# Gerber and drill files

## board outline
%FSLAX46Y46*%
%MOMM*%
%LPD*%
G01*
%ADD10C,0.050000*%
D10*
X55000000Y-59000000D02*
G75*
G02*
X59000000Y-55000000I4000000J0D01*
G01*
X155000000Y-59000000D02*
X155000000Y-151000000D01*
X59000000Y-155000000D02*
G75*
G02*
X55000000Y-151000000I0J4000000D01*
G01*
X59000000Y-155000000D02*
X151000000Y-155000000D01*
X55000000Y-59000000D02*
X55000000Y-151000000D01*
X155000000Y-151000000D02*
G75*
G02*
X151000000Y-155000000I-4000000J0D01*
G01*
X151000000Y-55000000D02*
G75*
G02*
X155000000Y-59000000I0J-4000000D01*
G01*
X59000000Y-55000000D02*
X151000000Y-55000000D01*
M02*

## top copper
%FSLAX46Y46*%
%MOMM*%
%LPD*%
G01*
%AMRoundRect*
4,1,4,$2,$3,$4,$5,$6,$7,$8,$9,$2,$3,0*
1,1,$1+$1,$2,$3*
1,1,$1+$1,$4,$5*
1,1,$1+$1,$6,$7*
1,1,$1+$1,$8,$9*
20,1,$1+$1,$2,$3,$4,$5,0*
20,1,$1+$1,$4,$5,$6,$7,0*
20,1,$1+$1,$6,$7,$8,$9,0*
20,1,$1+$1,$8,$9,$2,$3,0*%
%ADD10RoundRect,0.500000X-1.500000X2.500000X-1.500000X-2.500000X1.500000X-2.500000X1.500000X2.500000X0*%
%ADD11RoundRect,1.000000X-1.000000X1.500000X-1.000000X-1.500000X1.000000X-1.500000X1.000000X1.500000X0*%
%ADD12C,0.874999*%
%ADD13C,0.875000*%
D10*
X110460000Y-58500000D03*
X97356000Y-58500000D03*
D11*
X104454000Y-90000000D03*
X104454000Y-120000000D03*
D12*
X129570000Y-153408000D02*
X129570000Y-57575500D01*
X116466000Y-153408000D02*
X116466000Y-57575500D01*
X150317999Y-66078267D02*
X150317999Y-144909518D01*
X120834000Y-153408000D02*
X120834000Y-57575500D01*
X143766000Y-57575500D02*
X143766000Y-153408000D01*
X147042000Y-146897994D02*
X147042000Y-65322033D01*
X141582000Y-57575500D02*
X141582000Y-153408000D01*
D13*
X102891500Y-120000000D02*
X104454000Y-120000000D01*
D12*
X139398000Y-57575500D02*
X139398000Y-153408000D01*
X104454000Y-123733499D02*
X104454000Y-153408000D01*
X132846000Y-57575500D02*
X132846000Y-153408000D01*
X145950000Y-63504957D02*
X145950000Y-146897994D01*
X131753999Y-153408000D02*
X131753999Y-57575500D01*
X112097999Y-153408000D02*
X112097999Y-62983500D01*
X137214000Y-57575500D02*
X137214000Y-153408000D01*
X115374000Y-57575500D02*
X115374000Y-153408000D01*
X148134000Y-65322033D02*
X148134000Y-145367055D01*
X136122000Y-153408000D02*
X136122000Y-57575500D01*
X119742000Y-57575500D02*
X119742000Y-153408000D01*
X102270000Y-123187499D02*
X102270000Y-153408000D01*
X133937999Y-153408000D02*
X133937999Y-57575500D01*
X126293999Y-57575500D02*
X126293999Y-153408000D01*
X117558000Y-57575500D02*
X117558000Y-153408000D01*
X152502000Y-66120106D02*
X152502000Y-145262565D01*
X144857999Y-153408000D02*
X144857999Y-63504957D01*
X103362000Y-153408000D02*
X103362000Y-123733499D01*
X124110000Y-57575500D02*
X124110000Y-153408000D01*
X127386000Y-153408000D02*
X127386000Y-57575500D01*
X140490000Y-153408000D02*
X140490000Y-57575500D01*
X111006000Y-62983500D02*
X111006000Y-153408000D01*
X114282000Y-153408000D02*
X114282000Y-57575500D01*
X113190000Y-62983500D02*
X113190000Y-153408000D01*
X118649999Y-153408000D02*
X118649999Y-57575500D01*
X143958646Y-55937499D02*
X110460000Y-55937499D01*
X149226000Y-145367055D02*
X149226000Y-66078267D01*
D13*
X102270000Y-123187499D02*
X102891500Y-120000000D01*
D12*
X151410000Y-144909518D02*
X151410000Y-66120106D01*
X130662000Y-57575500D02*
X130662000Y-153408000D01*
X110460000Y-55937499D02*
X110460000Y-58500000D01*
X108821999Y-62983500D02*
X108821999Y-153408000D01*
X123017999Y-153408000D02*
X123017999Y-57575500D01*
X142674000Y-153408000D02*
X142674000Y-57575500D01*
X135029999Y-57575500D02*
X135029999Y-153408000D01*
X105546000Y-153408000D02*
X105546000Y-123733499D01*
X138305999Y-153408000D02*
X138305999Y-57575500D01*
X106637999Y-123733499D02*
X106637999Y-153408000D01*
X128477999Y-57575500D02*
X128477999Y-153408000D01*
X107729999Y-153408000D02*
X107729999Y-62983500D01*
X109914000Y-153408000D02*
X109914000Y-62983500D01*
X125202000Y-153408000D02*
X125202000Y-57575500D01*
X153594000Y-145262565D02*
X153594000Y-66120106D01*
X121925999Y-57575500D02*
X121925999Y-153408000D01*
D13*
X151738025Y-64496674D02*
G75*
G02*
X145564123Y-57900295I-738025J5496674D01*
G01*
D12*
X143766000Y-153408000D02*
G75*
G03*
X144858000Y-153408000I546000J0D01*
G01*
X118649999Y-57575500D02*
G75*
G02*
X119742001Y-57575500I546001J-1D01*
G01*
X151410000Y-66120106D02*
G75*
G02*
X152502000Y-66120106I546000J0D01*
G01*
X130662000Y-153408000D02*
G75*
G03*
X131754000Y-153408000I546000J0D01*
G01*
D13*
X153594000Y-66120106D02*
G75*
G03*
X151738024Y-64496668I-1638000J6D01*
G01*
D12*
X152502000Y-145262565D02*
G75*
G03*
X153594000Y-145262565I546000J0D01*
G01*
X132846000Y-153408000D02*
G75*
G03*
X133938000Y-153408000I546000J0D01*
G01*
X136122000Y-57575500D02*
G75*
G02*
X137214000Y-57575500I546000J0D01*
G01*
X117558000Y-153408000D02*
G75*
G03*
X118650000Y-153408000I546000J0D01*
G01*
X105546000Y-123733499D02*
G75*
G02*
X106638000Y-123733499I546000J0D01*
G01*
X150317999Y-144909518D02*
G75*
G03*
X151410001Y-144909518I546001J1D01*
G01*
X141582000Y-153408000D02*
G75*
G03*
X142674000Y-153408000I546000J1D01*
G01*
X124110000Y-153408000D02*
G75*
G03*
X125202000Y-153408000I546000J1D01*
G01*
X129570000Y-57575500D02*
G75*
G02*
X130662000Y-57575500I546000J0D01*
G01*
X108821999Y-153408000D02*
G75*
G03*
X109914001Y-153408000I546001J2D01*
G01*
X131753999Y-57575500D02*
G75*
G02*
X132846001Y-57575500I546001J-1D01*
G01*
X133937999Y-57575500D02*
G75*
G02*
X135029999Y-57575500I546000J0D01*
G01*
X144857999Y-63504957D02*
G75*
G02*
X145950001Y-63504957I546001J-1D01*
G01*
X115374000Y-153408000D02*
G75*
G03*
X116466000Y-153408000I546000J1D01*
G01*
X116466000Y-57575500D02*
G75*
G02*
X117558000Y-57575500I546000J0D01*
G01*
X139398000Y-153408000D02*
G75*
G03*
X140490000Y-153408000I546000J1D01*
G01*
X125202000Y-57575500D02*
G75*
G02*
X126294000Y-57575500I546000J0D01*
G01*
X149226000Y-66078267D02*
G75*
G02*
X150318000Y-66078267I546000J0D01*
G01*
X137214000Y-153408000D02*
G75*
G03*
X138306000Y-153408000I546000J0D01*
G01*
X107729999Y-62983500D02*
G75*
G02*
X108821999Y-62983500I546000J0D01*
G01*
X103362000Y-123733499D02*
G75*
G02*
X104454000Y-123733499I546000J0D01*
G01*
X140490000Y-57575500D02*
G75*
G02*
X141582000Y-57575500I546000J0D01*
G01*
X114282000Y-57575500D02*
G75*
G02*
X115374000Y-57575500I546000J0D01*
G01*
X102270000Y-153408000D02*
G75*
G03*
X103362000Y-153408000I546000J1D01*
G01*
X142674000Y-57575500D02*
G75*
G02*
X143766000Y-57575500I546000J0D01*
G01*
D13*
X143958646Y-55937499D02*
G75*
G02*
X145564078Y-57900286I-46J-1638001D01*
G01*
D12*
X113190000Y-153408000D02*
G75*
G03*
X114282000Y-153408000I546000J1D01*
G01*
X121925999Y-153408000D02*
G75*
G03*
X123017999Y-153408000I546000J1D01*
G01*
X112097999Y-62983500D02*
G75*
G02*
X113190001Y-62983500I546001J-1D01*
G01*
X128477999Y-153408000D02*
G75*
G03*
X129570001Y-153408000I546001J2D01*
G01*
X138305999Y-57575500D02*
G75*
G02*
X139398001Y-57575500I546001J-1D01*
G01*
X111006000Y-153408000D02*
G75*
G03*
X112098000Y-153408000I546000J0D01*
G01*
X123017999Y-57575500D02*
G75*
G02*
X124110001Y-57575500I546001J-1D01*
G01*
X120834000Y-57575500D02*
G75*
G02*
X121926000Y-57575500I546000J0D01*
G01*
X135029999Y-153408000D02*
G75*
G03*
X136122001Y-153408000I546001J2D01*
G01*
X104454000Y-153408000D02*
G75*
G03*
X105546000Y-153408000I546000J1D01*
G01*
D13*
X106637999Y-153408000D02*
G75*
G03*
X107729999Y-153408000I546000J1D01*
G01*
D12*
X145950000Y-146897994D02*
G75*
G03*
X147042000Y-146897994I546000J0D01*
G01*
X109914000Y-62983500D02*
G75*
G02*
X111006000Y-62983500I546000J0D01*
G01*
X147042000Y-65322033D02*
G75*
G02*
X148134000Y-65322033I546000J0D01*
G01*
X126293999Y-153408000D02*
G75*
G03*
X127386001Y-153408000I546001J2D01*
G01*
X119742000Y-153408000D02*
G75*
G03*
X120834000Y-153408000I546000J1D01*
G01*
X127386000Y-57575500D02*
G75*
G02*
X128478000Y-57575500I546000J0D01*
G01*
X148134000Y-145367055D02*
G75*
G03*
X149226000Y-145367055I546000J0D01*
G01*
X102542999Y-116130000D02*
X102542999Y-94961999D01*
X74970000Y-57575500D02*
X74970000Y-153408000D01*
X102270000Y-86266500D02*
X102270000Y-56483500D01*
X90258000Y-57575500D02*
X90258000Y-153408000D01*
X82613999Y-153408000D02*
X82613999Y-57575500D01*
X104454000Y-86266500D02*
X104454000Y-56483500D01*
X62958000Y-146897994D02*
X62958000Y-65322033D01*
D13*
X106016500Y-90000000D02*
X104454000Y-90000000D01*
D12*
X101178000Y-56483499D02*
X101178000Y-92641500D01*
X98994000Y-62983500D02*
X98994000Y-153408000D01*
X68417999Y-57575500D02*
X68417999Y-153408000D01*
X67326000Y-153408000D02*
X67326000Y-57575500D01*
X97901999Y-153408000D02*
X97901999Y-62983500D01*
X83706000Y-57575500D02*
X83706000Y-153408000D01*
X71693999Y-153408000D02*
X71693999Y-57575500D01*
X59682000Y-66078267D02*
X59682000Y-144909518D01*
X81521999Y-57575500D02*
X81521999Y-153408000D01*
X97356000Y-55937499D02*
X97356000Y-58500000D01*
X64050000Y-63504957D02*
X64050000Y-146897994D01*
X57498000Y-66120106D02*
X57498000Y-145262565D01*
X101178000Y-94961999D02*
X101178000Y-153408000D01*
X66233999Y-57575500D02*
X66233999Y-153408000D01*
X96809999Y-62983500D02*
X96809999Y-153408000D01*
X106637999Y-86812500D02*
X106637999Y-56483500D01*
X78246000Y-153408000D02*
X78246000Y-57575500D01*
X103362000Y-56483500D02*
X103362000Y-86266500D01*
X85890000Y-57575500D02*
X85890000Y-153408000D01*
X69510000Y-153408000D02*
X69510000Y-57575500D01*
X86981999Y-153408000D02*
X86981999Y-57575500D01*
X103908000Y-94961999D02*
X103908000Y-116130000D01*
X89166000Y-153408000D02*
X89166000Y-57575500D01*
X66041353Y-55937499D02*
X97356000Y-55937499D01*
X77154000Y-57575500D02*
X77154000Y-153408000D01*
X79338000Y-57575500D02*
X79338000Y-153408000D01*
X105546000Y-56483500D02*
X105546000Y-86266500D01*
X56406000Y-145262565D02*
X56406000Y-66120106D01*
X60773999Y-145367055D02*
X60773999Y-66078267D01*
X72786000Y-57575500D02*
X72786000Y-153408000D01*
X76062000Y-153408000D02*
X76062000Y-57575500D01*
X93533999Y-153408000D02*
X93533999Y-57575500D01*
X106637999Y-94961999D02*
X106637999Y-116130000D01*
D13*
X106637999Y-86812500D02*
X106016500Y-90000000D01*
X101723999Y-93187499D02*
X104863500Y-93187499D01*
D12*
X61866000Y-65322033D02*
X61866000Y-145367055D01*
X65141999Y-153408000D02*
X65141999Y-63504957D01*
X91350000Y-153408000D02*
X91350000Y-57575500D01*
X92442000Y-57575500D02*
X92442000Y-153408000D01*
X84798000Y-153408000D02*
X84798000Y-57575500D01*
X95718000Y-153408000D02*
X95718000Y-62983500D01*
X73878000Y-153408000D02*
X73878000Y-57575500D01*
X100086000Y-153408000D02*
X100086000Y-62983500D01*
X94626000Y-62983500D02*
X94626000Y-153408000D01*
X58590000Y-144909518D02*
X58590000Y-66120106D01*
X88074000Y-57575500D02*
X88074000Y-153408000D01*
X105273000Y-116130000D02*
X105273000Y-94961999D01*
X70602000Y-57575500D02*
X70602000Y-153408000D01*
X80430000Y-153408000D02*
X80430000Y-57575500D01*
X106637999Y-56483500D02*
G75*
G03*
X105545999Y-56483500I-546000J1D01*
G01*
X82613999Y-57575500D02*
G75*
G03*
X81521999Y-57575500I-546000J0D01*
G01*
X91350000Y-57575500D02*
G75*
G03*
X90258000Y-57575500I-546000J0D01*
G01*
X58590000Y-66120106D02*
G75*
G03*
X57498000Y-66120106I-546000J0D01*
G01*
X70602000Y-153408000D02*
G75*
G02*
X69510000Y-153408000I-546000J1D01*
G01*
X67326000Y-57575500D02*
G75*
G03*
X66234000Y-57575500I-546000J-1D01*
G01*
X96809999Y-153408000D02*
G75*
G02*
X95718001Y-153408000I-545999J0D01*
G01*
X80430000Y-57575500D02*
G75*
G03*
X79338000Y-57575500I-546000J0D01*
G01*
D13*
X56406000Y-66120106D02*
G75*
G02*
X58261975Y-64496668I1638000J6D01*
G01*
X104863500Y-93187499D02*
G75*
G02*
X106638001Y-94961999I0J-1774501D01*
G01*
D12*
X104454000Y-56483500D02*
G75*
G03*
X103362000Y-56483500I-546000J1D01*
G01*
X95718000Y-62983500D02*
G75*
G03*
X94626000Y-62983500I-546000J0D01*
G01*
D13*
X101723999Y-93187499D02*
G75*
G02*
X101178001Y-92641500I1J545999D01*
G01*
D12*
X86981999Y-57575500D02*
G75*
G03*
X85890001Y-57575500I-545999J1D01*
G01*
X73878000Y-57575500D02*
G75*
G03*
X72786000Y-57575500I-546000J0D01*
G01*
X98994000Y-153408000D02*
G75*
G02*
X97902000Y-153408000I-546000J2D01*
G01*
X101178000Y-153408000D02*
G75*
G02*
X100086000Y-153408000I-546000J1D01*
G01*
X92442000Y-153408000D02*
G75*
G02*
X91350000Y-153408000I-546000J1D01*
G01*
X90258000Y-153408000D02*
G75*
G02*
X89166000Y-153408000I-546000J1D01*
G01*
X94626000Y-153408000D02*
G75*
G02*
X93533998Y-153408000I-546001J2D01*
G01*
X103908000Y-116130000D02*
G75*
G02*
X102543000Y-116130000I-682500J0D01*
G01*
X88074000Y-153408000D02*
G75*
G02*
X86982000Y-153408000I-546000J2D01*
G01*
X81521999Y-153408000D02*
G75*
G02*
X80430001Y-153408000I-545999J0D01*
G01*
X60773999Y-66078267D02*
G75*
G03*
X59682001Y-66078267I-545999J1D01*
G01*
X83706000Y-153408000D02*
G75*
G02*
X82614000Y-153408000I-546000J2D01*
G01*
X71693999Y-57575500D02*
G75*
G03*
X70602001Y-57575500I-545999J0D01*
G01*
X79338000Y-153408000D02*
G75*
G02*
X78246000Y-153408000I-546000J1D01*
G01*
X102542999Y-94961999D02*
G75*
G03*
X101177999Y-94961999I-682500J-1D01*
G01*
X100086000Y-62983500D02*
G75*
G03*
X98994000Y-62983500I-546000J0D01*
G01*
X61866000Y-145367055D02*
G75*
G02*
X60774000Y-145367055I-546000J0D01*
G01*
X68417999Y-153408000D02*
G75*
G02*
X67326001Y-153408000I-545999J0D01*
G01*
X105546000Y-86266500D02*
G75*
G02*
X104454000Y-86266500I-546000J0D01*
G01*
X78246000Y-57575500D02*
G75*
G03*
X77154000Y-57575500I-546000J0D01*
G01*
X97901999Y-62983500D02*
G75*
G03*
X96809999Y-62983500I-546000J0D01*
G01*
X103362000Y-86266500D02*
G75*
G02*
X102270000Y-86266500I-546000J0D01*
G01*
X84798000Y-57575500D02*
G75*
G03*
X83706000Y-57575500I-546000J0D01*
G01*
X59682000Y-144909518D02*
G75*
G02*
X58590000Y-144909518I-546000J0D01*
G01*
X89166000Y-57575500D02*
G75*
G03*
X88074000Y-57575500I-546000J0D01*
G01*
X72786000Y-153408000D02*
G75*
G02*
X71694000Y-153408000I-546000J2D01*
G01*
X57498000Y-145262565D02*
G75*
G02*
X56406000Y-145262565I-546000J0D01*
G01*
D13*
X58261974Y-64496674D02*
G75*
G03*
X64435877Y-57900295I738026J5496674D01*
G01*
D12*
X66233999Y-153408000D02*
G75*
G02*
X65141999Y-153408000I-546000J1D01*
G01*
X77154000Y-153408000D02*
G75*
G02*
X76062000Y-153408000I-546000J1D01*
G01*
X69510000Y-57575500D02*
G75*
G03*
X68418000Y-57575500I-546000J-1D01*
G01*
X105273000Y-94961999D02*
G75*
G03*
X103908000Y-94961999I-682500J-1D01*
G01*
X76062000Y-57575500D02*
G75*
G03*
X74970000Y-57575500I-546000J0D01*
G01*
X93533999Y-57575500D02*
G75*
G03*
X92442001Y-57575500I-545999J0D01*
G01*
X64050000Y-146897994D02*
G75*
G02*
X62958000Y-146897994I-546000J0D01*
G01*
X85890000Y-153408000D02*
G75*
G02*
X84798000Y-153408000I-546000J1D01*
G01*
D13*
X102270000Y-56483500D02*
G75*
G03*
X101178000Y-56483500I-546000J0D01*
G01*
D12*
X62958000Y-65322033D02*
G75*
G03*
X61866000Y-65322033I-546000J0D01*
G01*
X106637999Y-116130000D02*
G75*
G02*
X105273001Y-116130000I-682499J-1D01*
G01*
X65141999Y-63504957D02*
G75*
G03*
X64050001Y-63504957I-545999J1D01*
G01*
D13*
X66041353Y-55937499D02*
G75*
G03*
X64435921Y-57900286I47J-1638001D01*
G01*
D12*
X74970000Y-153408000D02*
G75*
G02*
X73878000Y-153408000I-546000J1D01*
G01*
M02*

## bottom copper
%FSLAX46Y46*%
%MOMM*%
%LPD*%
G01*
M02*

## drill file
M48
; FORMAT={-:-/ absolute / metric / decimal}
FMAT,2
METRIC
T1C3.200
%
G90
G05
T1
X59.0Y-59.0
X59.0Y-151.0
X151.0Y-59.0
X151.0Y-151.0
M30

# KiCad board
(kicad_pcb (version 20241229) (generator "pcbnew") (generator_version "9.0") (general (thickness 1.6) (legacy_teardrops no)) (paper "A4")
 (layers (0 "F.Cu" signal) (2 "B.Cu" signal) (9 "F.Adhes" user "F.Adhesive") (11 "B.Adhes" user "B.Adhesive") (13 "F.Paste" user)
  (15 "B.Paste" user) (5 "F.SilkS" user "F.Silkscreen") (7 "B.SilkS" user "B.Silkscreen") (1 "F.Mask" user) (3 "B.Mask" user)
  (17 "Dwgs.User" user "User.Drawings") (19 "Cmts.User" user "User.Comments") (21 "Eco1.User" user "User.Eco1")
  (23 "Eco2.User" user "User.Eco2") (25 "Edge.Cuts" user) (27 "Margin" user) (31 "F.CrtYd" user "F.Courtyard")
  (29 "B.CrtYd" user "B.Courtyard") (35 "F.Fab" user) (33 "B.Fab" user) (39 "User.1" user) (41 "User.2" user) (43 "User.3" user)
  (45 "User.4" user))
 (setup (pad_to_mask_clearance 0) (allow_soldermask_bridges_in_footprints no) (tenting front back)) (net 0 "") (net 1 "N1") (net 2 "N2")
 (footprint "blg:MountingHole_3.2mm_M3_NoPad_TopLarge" (layer "F.Cu") (at 151 59)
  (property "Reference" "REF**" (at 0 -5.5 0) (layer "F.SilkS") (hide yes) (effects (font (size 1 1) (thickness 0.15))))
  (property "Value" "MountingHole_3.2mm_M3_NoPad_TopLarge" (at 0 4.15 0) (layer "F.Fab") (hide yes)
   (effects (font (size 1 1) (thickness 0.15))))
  (pad "" np_thru_hole circle (at 0 0) (size 7.6 7.6) (drill 3.2) (layers) (zone_connect 2)))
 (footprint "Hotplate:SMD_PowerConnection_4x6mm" (layer "F.Cu") (at 110.46 58.5 -90)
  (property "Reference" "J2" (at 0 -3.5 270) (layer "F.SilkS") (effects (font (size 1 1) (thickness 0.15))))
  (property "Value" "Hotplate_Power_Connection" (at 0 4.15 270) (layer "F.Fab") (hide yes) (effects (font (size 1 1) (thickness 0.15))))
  (pad "1" smd roundrect (at 0 0 270) (size 6 4) (layers "F.Cu" "F.Mask" "F.Paste") (roundrect_rratio 0.125) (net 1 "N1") (zone_connect 2)))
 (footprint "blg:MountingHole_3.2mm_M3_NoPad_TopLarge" (layer "F.Cu") (at 59 151)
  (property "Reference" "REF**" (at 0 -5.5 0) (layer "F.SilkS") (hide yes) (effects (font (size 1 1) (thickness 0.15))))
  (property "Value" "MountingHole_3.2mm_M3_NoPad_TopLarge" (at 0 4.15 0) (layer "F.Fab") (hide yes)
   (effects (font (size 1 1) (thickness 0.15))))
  (pad "" np_thru_hole circle (at 0 0) (size 7.6 7.6) (drill 3.2) (layers) (zone_connect 2)))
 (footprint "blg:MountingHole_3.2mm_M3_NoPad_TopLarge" (layer "F.Cu") (at 151 151)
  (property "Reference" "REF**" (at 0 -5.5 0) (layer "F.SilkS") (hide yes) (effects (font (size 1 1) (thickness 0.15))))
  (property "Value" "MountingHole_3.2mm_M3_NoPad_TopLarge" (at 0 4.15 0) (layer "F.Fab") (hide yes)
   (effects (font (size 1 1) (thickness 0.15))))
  (pad "" np_thru_hole circle (at 0 0) (size 7.6 7.6) (drill 3.2) (layers) (zone_connect 2)))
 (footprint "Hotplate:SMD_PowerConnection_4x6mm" (layer "F.Cu") (at 97.356 58.5 -90)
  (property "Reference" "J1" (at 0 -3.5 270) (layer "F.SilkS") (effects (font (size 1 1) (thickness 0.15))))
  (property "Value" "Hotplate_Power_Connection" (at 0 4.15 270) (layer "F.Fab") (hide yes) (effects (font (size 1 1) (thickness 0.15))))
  (pad "1" smd roundrect (at 0 0 270) (size 6 4) (layers "F.Cu" "F.Mask" "F.Paste") (roundrect_rratio 0.125) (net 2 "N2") (zone_connect 2)))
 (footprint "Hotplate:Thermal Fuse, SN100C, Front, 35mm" (layer "F.Cu") (at 104.454 105 -90)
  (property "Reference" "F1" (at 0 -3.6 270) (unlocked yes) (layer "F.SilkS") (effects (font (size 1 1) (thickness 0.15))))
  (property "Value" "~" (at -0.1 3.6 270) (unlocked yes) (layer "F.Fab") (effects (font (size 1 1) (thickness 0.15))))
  (pad "1" smd roundrect (at -15 0 270) (size 5 4) (layers "F.Cu" "F.Mask") (roundrect_rratio 0.25) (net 2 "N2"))
  (pad "2" smd roundrect (at 15 0 270) (size 5 4) (layers "F.Cu" "F.Mask") (roundrect_rratio 0.25) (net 1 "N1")))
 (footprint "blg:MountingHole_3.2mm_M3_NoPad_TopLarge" (layer "F.Cu") (at 59 59)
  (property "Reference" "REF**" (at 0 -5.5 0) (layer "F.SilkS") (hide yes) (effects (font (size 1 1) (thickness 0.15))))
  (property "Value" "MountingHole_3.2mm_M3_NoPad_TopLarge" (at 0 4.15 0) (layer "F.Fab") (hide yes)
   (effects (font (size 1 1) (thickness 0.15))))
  (pad "" np_thru_hole circle (at 0 0) (size 7.6 7.6) (drill 3.2) (layers) (zone_connect 2)))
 (gr_arc (start 55 59) (mid 56.171573 56.171573) (end 59 55) (stroke (width 0.05) (type solid)) (layer "Edge.Cuts"))
 (gr_line (start 155 59) (end 155 151) (stroke (width 0.05) (type default)) (layer "Edge.Cuts"))
 (gr_arc (start 59 155) (mid 56.171573 153.828427) (end 55 151) (stroke (width 0.05) (type solid)) (layer "Edge.Cuts"))
 (gr_line (start 59 155) (end 151 155) (stroke (width 0.05) (type default)) (layer "Edge.Cuts"))
 (gr_line (start 55 59) (end 55 151) (stroke (width 0.05) (type default)) (layer "Edge.Cuts"))
 (gr_arc (start 155 151) (mid 153.828427 153.828427) (end 151 155) (stroke (width 0.05) (type solid)) (layer "Edge.Cuts"))
 (gr_arc (start 151 55) (mid 153.828427 56.171573) (end 155 59) (stroke (width 0.05) (type solid)) (layer "Edge.Cuts"))
 (gr_line (start 59 55) (end 151 55) (stroke (width 0.05) (type default)) (layer "Edge.Cuts"))
 (segment (start 129.57 153.408) (end 129.57 57.5755) (width 0.874999) (layer "F.Cu") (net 1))
 (segment (start 116.466 153.408) (end 116.466 57.5755) (width 0.874999) (layer "F.Cu") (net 1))
 (segment (start 150.317999 66.078267) (end 150.317999 144.909518) (width 0.874999) (layer "F.Cu") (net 1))
 (segment (start 120.834 153.408) (end 120.834 57.5755) (width 0.874999) (layer "F.Cu") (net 1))
 (segment (start 143.766 57.5755) (end 143.766 153.408) (width 0.874999) (layer "F.Cu") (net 1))
 (segment (start 147.042 146.897994) (end 147.042 65.322033) (width 0.874999) (layer "F.Cu") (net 1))
 (segment (start 141.582 57.5755) (end 141.582 153.408) (width 0.874999) (layer "F.Cu") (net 1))
 (segment (start 102.8915 120) (end 104.454 120) (width 0.875) (layer "F.Cu") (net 1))
 (segment (start 139.398 57.5755) (end 139.398 153.408) (width 0.874999) (layer "F.Cu") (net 1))
 (segment (start 104.454 123.733499) (end 104.454 153.408) (width 0.874999) (layer "F.Cu") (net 1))
 (segment (start 132.846 57.5755) (end 132.846 153.408) (width 0.874999) (layer "F.Cu") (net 1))
 (segment (start 145.95 63.504957) (end 145.95 146.897994) (width 0.874999) (layer "F.Cu") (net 1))
 (segment (start 131.753999 153.408) (end 131.753999 57.5755) (width 0.874999) (layer "F.Cu") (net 1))
 (segment (start 112.097999 153.408) (end 112.097999 62.9835) (width 0.874999) (layer "F.Cu") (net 1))
 (segment (start 137.214 57.5755) (end 137.214 153.408) (width 0.874999) (layer "F.Cu") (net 1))
 (segment (start 115.374 57.5755) (end 115.374 153.408) (width 0.874999) (layer "F.Cu") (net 1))
 (segment (start 148.134 65.322033) (end 148.134 145.367055) (width 0.874999) (layer "F.Cu") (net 1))
 (segment (start 136.122 153.408) (end 136.122 57.5755) (width 0.874999) (layer "F.Cu") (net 1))
 (segment (start 119.742 57.5755) (end 119.742 153.408) (width 0.874999) (layer "F.Cu") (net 1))
 (segment (start 102.27 123.187499) (end 102.27 153.408) (width 0.874999) (layer "F.Cu") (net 1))
 (segment (start 133.937999 153.408) (end 133.937999 57.5755) (width 0.874999) (layer "F.Cu") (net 1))
 (segment (start 126.293999 57.5755) (end 126.293999 153.408) (width 0.874999) (layer "F.Cu") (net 1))
 (segment (start 117.558 57.5755) (end 117.558 153.408) (width 0.874999) (layer "F.Cu") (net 1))
 (segment (start 152.502 66.120106) (end 152.502 145.262565) (width 0.874999) (layer "F.Cu") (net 1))
 (segment (start 144.857999 153.408) (end 144.857999 63.504957) (width 0.874999) (layer "F.Cu") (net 1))
 (segment (start 103.362 153.408) (end 103.362 123.733499) (width 0.874999) (layer "F.Cu") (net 1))
 (segment (start 124.11 57.5755) (end 124.11 153.408) (width 0.874999) (layer "F.Cu") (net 1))
 (segment (start 127.386 153.408) (end 127.386 57.5755) (width 0.874999) (layer "F.Cu") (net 1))
 (segment (start 140.49 153.408) (end 140.49 57.5755) (width 0.874999) (layer "F.Cu") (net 1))
 (segment (start 111.006 62.9835) (end 111.006 153.408) (width 0.874999) (layer "F.Cu") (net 1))
 (segment (start 114.282 153.408) (end 114.282 57.5755) (width 0.874999) (layer "F.Cu") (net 1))
 (segment (start 113.19 62.9835) (end 113.19 153.408) (width 0.874999) (layer "F.Cu") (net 1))
 (segment (start 118.649999 153.408) (end 118.649999 57.5755) (width 0.874999) (layer "F.Cu") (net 1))
 (segment (start 143.958646 55.937499) (end 110.46 55.937499) (width 0.874999) (layer "F.Cu") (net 1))
 (segment (start 149.226 145.367055) (end 149.226 66.078267) (width 0.874999) (layer "F.Cu") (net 1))
 (segment (start 102.27 123.187499) (end 102.8915 120) (width 0.875) (layer "F.Cu") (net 1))
 (segment (start 151.41 144.909518) (end 151.41 66.120106) (width 0.874999) (layer "F.Cu") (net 1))
 (segment (start 130.662 57.5755) (end 130.662 153.408) (width 0.874999) (layer "F.Cu") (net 1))
 (segment (start 110.46 55.937499) (end 110.46 58.5) (width 0.874999) (layer "F.Cu") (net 1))
 (segment (start 108.821999 62.9835) (end 108.821999 153.408) (width 0.874999) (layer "F.Cu") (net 1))
 (segment (start 123.017999 153.408) (end 123.017999 57.5755) (width 0.874999) (layer "F.Cu") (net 1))
 (segment (start 142.674 153.408) (end 142.674 57.5755) (width 0.874999) (layer "F.Cu") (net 1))
 (segment (start 135.029999 57.5755) (end 135.029999 153.408) (width 0.874999) (layer "F.Cu") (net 1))
 (segment (start 105.546 153.408) (end 105.546 123.733499) (width 0.874999) (layer "F.Cu") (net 1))
 (segment (start 138.305999 153.408) (end 138.305999 57.5755) (width 0.874999) (layer "F.Cu") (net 1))
 (segment (start 106.637999 123.733499) (end 106.637999 153.408) (width 0.874999) (layer "F.Cu") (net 1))
 (segment (start 128.477999 57.5755) (end 128.477999 153.408) (width 0.874999) (layer "F.Cu") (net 1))
 (segment (start 107.729999 153.408) (end 107.729999 62.9835) (width 0.874999) (layer "F.Cu") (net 1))
 (segment (start 109.914 153.408) (end 109.914 62.9835) (width 0.874999) (layer "F.Cu") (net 1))
 (segment (start 125.202 153.408) (end 125.202 57.5755) (width 0.874999) (layer "F.Cu") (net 1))
 (segment (start 153.594 145.262565) (end 153.594 66.120106) (width 0.874999) (layer "F.Cu") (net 1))
 (segment (start 121.925999 57.5755) (end 121.925999 153.408) (width 0.874999) (layer "F.Cu") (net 1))
 (arc (start 151.738025 64.496674) (mid 146.950863 62.789803) (end 145.564122 57.900295) (width 0.875) (layer "F.Cu") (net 1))
 (arc (start 143.766 153.408) (mid 144.311999 153.953999) (end 144.857999 153.408) (width 0.874999) (layer "F.Cu") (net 1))
 (arc (start 118.649999 57.5755) (mid 119.196 57.0295) (end 119.742 57.5755) (width 0.874999) (layer "F.Cu") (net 1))
 (arc (start 151.41 66.120106) (mid 151.956 65.574106) (end 152.502 66.120106) (width 0.874999) (layer "F.Cu") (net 1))
 (arc (start 130.662 153.408) (mid 131.208 153.953999) (end 131.753999 153.408) (width 0.874999) (layer "F.Cu") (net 1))
 (arc (start 153.594 66.120106) (mid 153.16814 65.018399) (end 151.738025 64.496674) (width 0.875) (layer "F.Cu") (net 1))
 (arc (start 152.502 145.262565) (mid 153.048 145.808565) (end 153.594 145.262565) (width 0.874999) (layer "F.Cu") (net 1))
 (arc (start 132.846 153.408) (mid 133.392 153.953999) (end 133.937999 153.408) (width 0.874999) (layer "F.Cu") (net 1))
 (arc (start 136.122 57.5755) (mid 136.667999 57.0295) (end 137.214 57.5755) (width 0.874999) (layer "F.Cu") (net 1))
 (arc (start 117.558 153.408) (mid 118.104 153.953999) (end 118.649999 153.408) (width 0.874999) (layer "F.Cu") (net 1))
 (arc (start 105.546 123.733499) (mid 106.092 123.187499) (end 106.637999 123.733499) (width 0.874999) (layer "F.Cu") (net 1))
 (arc (start 150.317999 144.909518) (mid 150.864 145.455518) (end 151.41 144.909518) (width 0.874999) (layer "F.Cu") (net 1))
 (arc (start 141.582 153.408) (mid 142.128 153.953999) (end 142.674 153.408) (width 0.874999) (layer "F.Cu") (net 1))
 (arc (start 124.11 153.408) (mid 124.655999 153.953999) (end 125.202 153.408) (width 0.874999) (layer "F.Cu") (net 1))
 (arc (start 129.57 57.5755) (mid 130.115999 57.0295) (end 130.662 57.5755) (width 0.874999) (layer "F.Cu") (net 1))
 (arc (start 108.821999 153.408) (mid 109.368 153.953999) (end 109.914 153.408) (width 0.874999) (layer "F.Cu") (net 1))
 (arc (start 131.753999 57.5755) (mid 132.3 57.0295) (end 132.846 57.5755) (width 0.874999) (layer "F.Cu") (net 1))
 (arc (start 133.937999 57.5755) (mid 134.483999 57.0295) (end 135.029999 57.5755) (width 0.874999) (layer "F.Cu") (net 1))
 (arc (start 144.857999 63.504957) (mid 145.404 62.958957) (end 145.95 63.504957) (width 0.874999) (layer "F.Cu") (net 1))
 (arc (start 115.374 153.408) (mid 115.92 153.953999) (end 116.466 153.408) (width 0.874999) (layer "F.Cu") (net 1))
 (arc (start 116.466 57.5755) (mid 117.011999 57.0295) (end 117.558 57.5755) (width 0.874999) (layer "F.Cu") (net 1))
 (arc (start 139.398 153.408) (mid 139.944 153.953999) (end 140.49 153.408) (width 0.874999) (layer "F.Cu") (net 1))
 (arc (start 125.202 57.5755) (mid 125.748 57.0295) (end 126.293999 57.5755) (width 0.874999) (layer "F.Cu") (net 1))
 (arc (start 149.226 66.078267) (mid 149.772 65.532267) (end 150.317999 66.078267) (width 0.874999) (layer "F.Cu") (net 1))
 (arc (start 137.214 153.408) (mid 137.76 153.953999) (end 138.305999 153.408) (width 0.874999) (layer "F.Cu") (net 1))
 (arc (start 107.729999 62.9835) (mid 108.276 62.4375) (end 108.821999 62.9835) (width 0.874999) (layer "F.Cu") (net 1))
 (arc (start 103.362 123.733499) (mid 103.908 123.187499) (end 104.454 123.733499) (width 0.874999) (layer "F.Cu") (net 1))
 (arc (start 140.49 57.5755) (mid 141.036 57.0295) (end 141.582 57.5755) (width 0.874999) (layer "F.Cu") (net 1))
 (arc (start 114.282 57.5755) (mid 114.828 57.0295) (end 115.374 57.5755) (width 0.874999) (layer "F.Cu") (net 1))
 (arc (start 102.27 153.408) (mid 102.815999 153.953999) (end 103.362 153.408) (width 0.874999) (layer "F.Cu") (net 1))
 (arc (start 142.674 57.5755) (mid 143.22 57.0295) (end 143.766 57.5755) (width 0.874999) (layer "F.Cu") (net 1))
 (arc (start 143.958646 55.937499) (mid 145.22653 56.538429) (end 145.564122 57.900295) (width 0.875) (layer "F.Cu") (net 1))
 (arc (start 113.19 153.408) (mid 113.735999 153.953999) (end 114.282 153.408) (width 0.874999) (layer "F.Cu") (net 1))
 (arc (start 121.925999 153.408) (mid 122.472 153.953999) (end 123.017999 153.408) (width 0.874999) (layer "F.Cu") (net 1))
 (arc (start 112.097999 62.9835) (mid 112.643999 62.4375) (end 113.19 62.9835) (width 0.874999) (layer "F.Cu") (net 1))
 (arc (start 128.477999 153.408) (mid 129.024 153.953999) (end 129.57 153.408) (width 0.874999) (layer "F.Cu") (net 1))
 (arc (start 138.305999 57.5755) (mid 138.852 57.0295) (end 139.398 57.5755) (width 0.874999) (layer "F.Cu") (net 1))
 (arc (start 111.006 153.408) (mid 111.551999 153.953999) (end 112.097999 153.408) (width 0.874999) (layer "F.Cu") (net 1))
 (arc (start 123.017999 57.5755) (mid 123.564 57.0295) (end 124.11 57.5755) (width 0.874999) (layer "F.Cu") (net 1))
 (arc (start 120.834 57.5755) (mid 121.379999 57.0295) (end 121.925999 57.5755) (width 0.874999) (layer "F.Cu") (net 1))
 (arc (start 135.029999 153.408) (mid 135.576 153.953999) (end 136.122 153.408) (width 0.874999) (layer "F.Cu") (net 1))
 (arc (start 104.454 153.408) (mid 105 153.953999) (end 105.546 153.408) (width 0.874999) (layer "F.Cu") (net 1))
 (arc (start 106.637999 153.408) (mid 107.184 153.953999) (end 107.729999 153.408) (width 0.875) (layer "F.Cu") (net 1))
 (arc (start 145.95 146.897994) (mid 146.495999 147.443994) (end 147.042 146.897994) (width 0.874999) (layer "F.Cu") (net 1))
 (arc (start 109.914 62.9835) (mid 110.46 62.4375) (end 111.006 62.9835) (width 0.874999) (layer "F.Cu") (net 1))
 (arc (start 147.042 65.322033) (mid 147.588 64.776033) (end 148.134 65.322033) (width 0.874999) (layer "F.Cu") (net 1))
 (arc (start 126.293999 153.408) (mid 126.839999 153.953999) (end 127.386 153.408) (width 0.874999) (layer "F.Cu") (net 1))
 (arc (start 119.742 153.408) (mid 120.288 153.953999) (end 120.834 153.408) (width 0.874999) (layer "F.Cu") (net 1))
 (arc (start 127.386 57.5755) (mid 127.931999 57.0295) (end 128.477999 57.5755) (width 0.874999) (layer "F.Cu") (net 1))
 (arc (start 148.134 145.367055) (mid 148.68 145.913055) (end 149.226 145.367055) (width 0.874999) (layer "F.Cu") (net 1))
 (segment (start 102.542999 116.13) (end 102.542999 94.961999) (width 0.874999) (layer "F.Cu") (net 2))
 (segment (start 74.97 57.5755) (end 74.97 153.408) (width 0.874999) (layer "F.Cu") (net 2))
 (segment (start 102.27 86.2665) (end 102.27 56.4835) (width 0.874999) (layer "F.Cu") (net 2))
 (segment (start 90.258 57.5755) (end 90.258 153.408) (width 0.874999) (layer "F.Cu") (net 2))
 (segment (start 82.613999 153.408) (end 82.613999 57.5755) (width 0.874999) (layer "F.Cu") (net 2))
 (segment (start 104.454 86.2665) (end 104.454 56.4835) (width 0.874999) (layer "F.Cu") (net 2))
 (segment (start 62.958 146.897994) (end 62.958 65.322033) (width 0.874999) (layer "F.Cu") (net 2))
 (segment (start 106.0165 90) (end 104.454 90) (width 0.875) (layer "F.Cu") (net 2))
 (segment (start 101.178 56.483499) (end 101.178 92.6415) (width 0.874999) (layer "F.Cu") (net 2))
 (segment (start 98.994 62.9835) (end 98.994 153.408) (width 0.874999) (layer "F.Cu") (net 2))
 (segment (start 68.417999 57.5755) (end 68.417999 153.408) (width 0.874999) (layer "F.Cu") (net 2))
 (segment (start 67.326 153.408) (end 67.326 57.5755) (width 0.874999) (layer "F.Cu") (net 2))
 (segment (start 97.901999 153.408) (end 97.901999 62.9835) (width 0.874999) (layer "F.Cu") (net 2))
 (segment (start 83.706 57.5755) (end 83.706 153.408) (width 0.874999) (layer "F.Cu") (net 2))
 (segment (start 71.693999 153.408) (end 71.693999 57.5755) (width 0.874999) (layer "F.Cu") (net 2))
 (segment (start 59.682 66.078267) (end 59.682 144.909518) (width 0.874999) (layer "F.Cu") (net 2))
 (segment (start 81.521999 57.5755) (end 81.521999 153.408) (width 0.874999) (layer "F.Cu") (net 2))
 (segment (start 97.356 55.937499) (end 97.356 58.5) (width 0.874999) (layer "F.Cu") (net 2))
 (segment (start 64.05 63.504957) (end 64.05 146.897994) (width 0.874999) (layer "F.Cu") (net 2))
 (segment (start 57.498 66.120106) (end 57.498 145.262565) (width 0.874999) (layer "F.Cu") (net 2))
 (segment (start 101.178 94.961999) (end 101.178 153.408) (width 0.874999) (layer "F.Cu") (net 2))
 (segment (start 66.233999 57.5755) (end 66.233999 153.408) (width 0.874999) (layer "F.Cu") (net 2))
 (segment (start 96.809999 62.9835) (end 96.809999 153.408) (width 0.874999) (layer "F.Cu") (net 2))
 (segment (start 106.637999 86.8125) (end 106.637999 56.4835) (width 0.874999) (layer "F.Cu") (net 2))
 (segment (start 78.246 153.408) (end 78.246 57.5755) (width 0.874999) (layer "F.Cu") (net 2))
 (segment (start 103.362 56.4835) (end 103.362 86.2665) (width 0.874999) (layer "F.Cu") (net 2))
 (segment (start 85.89 57.5755) (end 85.89 153.408) (width 0.874999) (layer "F.Cu") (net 2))
 (segment (start 69.51 153.408) (end 69.51 57.5755) (width 0.874999) (layer "F.Cu") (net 2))
 (segment (start 86.981999 153.408) (end 86.981999 57.5755) (width 0.874999) (layer "F.Cu") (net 2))
 (segment (start 103.908 94.961999) (end 103.908 116.13) (width 0.874999) (layer "F.Cu") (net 2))
 (segment (start 89.166 153.408) (end 89.166 57.5755) (width 0.874999) (layer "F.Cu") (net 2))
 (segment (start 66.041353 55.937499) (end 97.356 55.937499) (width 0.874999) (layer "F.Cu") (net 2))
 (segment (start 77.154 57.5755) (end 77.154 153.408) (width 0.874999) (layer "F.Cu") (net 2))
 (segment (start 79.338 57.5755) (end 79.338 153.408) (width 0.874999) (layer "F.Cu") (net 2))
 (segment (start 105.546 56.4835) (end 105.546 86.2665) (width 0.874999) (layer "F.Cu") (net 2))
 (segment (start 56.406 145.262565) (end 56.406 66.120106) (width 0.874999) (layer "F.Cu") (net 2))
 (segment (start 60.773999 145.367055) (end 60.773999 66.078267) (width 0.874999) (layer "F.Cu") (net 2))
 (segment (start 72.786 57.5755) (end 72.786 153.408) (width 0.874999) (layer "F.Cu") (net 2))
 (segment (start 76.062 153.408) (end 76.062 57.5755) (width 0.874999) (layer "F.Cu") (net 2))
 (segment (start 93.533999 153.408) (end 93.533999 57.5755) (width 0.874999) (layer "F.Cu") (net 2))
 (segment (start 106.637999 94.961999) (end 106.637999 116.13) (width 0.874999) (layer "F.Cu") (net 2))
 (segment (start 106.637999 86.8125) (end 106.0165 90) (width 0.875) (layer "F.Cu") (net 2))
 (segment (start 101.723999 93.187499) (end 104.8635 93.187499) (width 0.875) (layer "F.Cu") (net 2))
 (segment (start 61.866 65.322033) (end 61.866 145.367055) (width 0.874999) (layer "F.Cu") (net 2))
 (segment (start 65.141999 153.408) (end 65.141999 63.504957) (width 0.874999) (layer "F.Cu") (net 2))
 (segment (start 91.35 153.408) (end 91.35 57.5755) (width 0.874999) (layer "F.Cu") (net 2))
 (segment (start 92.442 57.5755) (end 92.442 153.408) (width 0.874999) (layer "F.Cu") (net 2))
 (segment (start 84.798 153.408) (end 84.798 57.5755) (width 0.874999) (layer "F.Cu") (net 2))
 (segment (start 95.718 153.408) (end 95.718 62.9835) (width 0.874999) (layer "F.Cu") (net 2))
 (segment (start 73.878 153.408) (end 73.878 57.5755) (width 0.874999) (layer "F.Cu") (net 2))
 (segment (start 100.086 153.408) (end 100.086 62.9835) (width 0.874999) (layer "F.Cu") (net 2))
 (segment (start 94.626 62.9835) (end 94.626 153.408) (width 0.874999) (layer "F.Cu") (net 2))
 (segment (start 58.59 144.909518) (end 58.59 66.120106) (width 0.874999) (layer "F.Cu") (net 2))
 (segment (start 88.074 57.5755) (end 88.074 153.408) (width 0.874999) (layer "F.Cu") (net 2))
 (segment (start 105.273 116.13) (end 105.273 94.961999) (width 0.874999) (layer "F.Cu") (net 2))
 (segment (start 70.602 57.5755) (end 70.602 153.408) (width 0.874999) (layer "F.Cu") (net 2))
 (segment (start 80.43 153.408) (end 80.43 57.5755) (width 0.874999) (layer "F.Cu") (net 2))
 (arc (start 106.637999 56.4835) (mid 106.092 55.937499) (end 105.546 56.4835) (width 0.874999) (layer "F.Cu") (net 2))
 (arc (start 82.613999 57.5755) (mid 82.068 57.0295) (end 81.521999 57.5755) (width 0.874999) (layer "F.Cu") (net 2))
 (arc (start 91.35 57.5755) (mid 90.804 57.0295) (end 90.258 57.5755) (width 0.874999) (layer "F.Cu") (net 2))
 (arc (start 58.59 66.120106) (mid 58.044 65.574106) (end 57.498 66.120106) (width 0.874999) (layer "F.Cu") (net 2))
 (arc (start 70.602 153.408) (mid 70.056 153.953999) (end 69.51 153.408) (width 0.874999) (layer "F.Cu") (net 2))
 (arc (start 67.326 57.5755) (mid 66.779999 57.0295) (end 66.233999 57.5755) (width 0.874999) (layer "F.Cu") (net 2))
 (arc (start 96.809999 153.408) (mid 96.264 153.953999) (end 95.718 153.408) (width 0.874999) (layer "F.Cu") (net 2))
 (arc (start 80.43 57.5755) (mid 79.884 57.0295) (end 79.338 57.5755) (width 0.874999) (layer "F.Cu") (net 2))
 (arc (start 56.406 66.120106) (mid 56.831859 65.018399) (end 58.261974 64.496674) (width 0.875) (layer "F.Cu") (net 2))
 (arc (start 104.8635 93.187499) (mid 106.11826 93.707239) (end 106.637999 94.961999) (width 0.875) (layer "F.Cu") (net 2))
 (arc (start 104.454 56.4835) (mid 103.908 55.937499) (end 103.362 56.4835) (width 0.874999) (layer "F.Cu") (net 2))
 (arc (start 95.718 62.9835) (mid 95.172 62.4375) (end 94.626 62.9835) (width 0.874999) (layer "F.Cu") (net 2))
 (arc (start 101.723999 93.187499) (mid 101.337919 93.02758) (end 101.178 92.6415) (width 0.875) (layer "F.Cu") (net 2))
 (arc (start 86.981999 57.5755) (mid 86.436 57.0295) (end 85.89 57.5755) (width 0.874999) (layer "F.Cu") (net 2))
 (arc (start 73.878 57.5755) (mid 73.332 57.0295) (end 72.786 57.5755) (width 0.874999) (layer "F.Cu") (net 2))
 (arc (start 98.994 153.408) (mid 98.448 153.953999) (end 97.901999 153.408) (width 0.874999) (layer "F.Cu") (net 2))
 (arc (start 101.178 153.408) (mid 100.632 153.953999) (end 100.086 153.408) (width 0.874999) (layer "F.Cu") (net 2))
 (arc (start 92.442 153.408) (mid 91.895999 153.953999) (end 91.35 153.408) (width 0.874999) (layer "F.Cu") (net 2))
 (arc (start 90.258 153.408) (mid 89.712 153.953999) (end 89.166 153.408) (width 0.874999) (layer "F.Cu") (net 2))
 (arc (start 94.626 153.408) (mid 94.08 153.953999) (end 93.533999 153.408) (width 0.874999) (layer "F.Cu") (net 2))
 (arc (start 103.908 116.13) (mid 103.2255 116.8125) (end 102.542999 116.13) (width 0.874999) (layer "F.Cu") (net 2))
 (arc (start 88.074 153.408) (mid 87.527999 153.953999) (end 86.981999 153.408) (width 0.874999) (layer "F.Cu") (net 2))
 (arc (start 81.521999 153.408) (mid 80.976 153.953999) (end 80.43 153.408) (width 0.874999) (layer "F.Cu") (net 2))
 (arc (start 60.773999 66.078267) (mid 60.227999 65.532267) (end 59.682 66.078267) (width 0.874999) (layer "F.Cu") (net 2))
 (arc (start 83.706 153.408) (mid 83.16 153.953999) (end 82.613999 153.408) (width 0.874999) (layer "F.Cu") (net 2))
 (arc (start 71.693999 57.5755) (mid 71.148 57.0295) (end 70.602 57.5755) (width 0.874999) (layer "F.Cu") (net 2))
 (arc (start 79.338 153.408) (mid 78.792 153.953999) (end 78.246 153.408) (width 0.874999) (layer "F.Cu") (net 2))
 (arc (start 102.542999 94.961999) (mid 101.860499 94.2795) (end 101.178 94.961999) (width 0.874999) (layer "F.Cu") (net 2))
 (arc (start 100.086 62.9835) (mid 99.539999 62.4375) (end 98.994 62.9835) (width 0.874999) (layer "F.Cu") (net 2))
 (arc (start 61.866 145.367055) (mid 61.32 145.913055) (end 60.773999 145.367055) (width 0.874999) (layer "F.Cu") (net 2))
 (arc (start 68.417999 153.408) (mid 67.872 153.953999) (end 67.326 153.408) (width 0.874999) (layer "F.Cu") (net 2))
 (arc (start 105.546 86.2665) (mid 105 86.8125) (end 104.454 86.2665) (width 0.874999) (layer "F.Cu") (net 2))
 (arc (start 78.246 57.5755) (mid 77.699999 57.0295) (end 77.154 57.5755) (width 0.874999) (layer "F.Cu") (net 2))
 (arc (start 97.901999 62.9835) (mid 97.356 62.4375) (end 96.809999 62.9835) (width 0.874999) (layer "F.Cu") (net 2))
 (arc (start 103.362 86.2665) (mid 102.815999 86.8125) (end 102.27 86.2665) (width 0.874999) (layer "F.Cu") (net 2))
 (arc (start 84.798 57.5755) (mid 84.252 57.0295) (end 83.706 57.5755) (width 0.874999) (layer "F.Cu") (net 2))
 (arc (start 59.682 144.909518) (mid 59.135999 145.455518) (end 58.59 144.909518) (width 0.874999) (layer "F.Cu") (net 2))
 (arc (start 89.166 57.5755) (mid 88.619999 57.0295) (end 88.074 57.5755) (width 0.874999) (layer "F.Cu") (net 2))
 (arc (start 72.786 153.408) (mid 72.24 153.953999) (end 71.693999 153.408) (width 0.874999) (layer "F.Cu") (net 2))
 (arc (start 57.498 145.262565) (mid 56.952 145.808565) (end 56.406 145.262565) (width 0.874999) (layer "F.Cu") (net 2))
 (arc (start 58.261974 64.496674) (mid 63.049136 62.789803) (end 64.435877 57.900295) (width 0.875) (layer "F.Cu") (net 2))
 (arc (start 66.233999 153.408) (mid 65.688 153.953999) (end 65.141999 153.408) (width 0.874999) (layer "F.Cu") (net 2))
 (arc (start 77.154 153.408) (mid 76.607999 153.953999) (end 76.062 153.408) (width 0.874999) (layer "F.Cu") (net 2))
 (arc (start 69.51 57.5755) (mid 68.964 57.0295) (end 68.417999 57.5755) (width 0.874999) (layer "F.Cu") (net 2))
 (arc (start 105.273 94.961999) (mid 104.590499 94.2795) (end 103.908 94.961999) (width 0.874999) (layer "F.Cu") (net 2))
 (arc (start 76.062 57.5755) (mid 75.516 57.0295) (end 74.97 57.5755) (width 0.874999) (layer "F.Cu") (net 2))
 (arc (start 93.533999 57.5755) (mid 92.988 57.0295) (end 92.442 57.5755) (width 0.874999) (layer "F.Cu") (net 2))
 (arc (start 64.05 146.897994) (mid 63.503999 147.443994) (end 62.958 146.897994) (width 0.874999) (layer "F.Cu") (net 2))
 (arc (start 85.89 153.408) (mid 85.344 153.953999) (end 84.798 153.408) (width 0.874999) (layer "F.Cu") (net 2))
 (arc (start 102.27 56.4835) (mid 101.723999 55.9375) (end 101.178 56.4835) (width 0.875) (layer "F.Cu") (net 2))
 (arc (start 62.958 65.322033) (mid 62.411999 64.776033) (end 61.866 65.322033) (width 0.874999) (layer "F.Cu") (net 2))
 (arc (start 106.637999 116.13) (mid 105.9555 116.8125) (end 105.273 116.13) (width 0.874999) (layer "F.Cu") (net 2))
 (arc (start 65.141999 63.504957) (mid 64.596 62.958957) (end 64.05 63.504957) (width 0.874999) (layer "F.Cu") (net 2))
 (arc (start 66.041353 55.937499) (mid 64.773469 56.538429) (end 64.435877 57.900295) (width 0.875) (layer "F.Cu") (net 2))
 (arc (start 74.97 153.408) (mid 74.423999 153.953999) (end 73.878 153.408) (width 0.874999) (layer "F.Cu") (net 2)))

